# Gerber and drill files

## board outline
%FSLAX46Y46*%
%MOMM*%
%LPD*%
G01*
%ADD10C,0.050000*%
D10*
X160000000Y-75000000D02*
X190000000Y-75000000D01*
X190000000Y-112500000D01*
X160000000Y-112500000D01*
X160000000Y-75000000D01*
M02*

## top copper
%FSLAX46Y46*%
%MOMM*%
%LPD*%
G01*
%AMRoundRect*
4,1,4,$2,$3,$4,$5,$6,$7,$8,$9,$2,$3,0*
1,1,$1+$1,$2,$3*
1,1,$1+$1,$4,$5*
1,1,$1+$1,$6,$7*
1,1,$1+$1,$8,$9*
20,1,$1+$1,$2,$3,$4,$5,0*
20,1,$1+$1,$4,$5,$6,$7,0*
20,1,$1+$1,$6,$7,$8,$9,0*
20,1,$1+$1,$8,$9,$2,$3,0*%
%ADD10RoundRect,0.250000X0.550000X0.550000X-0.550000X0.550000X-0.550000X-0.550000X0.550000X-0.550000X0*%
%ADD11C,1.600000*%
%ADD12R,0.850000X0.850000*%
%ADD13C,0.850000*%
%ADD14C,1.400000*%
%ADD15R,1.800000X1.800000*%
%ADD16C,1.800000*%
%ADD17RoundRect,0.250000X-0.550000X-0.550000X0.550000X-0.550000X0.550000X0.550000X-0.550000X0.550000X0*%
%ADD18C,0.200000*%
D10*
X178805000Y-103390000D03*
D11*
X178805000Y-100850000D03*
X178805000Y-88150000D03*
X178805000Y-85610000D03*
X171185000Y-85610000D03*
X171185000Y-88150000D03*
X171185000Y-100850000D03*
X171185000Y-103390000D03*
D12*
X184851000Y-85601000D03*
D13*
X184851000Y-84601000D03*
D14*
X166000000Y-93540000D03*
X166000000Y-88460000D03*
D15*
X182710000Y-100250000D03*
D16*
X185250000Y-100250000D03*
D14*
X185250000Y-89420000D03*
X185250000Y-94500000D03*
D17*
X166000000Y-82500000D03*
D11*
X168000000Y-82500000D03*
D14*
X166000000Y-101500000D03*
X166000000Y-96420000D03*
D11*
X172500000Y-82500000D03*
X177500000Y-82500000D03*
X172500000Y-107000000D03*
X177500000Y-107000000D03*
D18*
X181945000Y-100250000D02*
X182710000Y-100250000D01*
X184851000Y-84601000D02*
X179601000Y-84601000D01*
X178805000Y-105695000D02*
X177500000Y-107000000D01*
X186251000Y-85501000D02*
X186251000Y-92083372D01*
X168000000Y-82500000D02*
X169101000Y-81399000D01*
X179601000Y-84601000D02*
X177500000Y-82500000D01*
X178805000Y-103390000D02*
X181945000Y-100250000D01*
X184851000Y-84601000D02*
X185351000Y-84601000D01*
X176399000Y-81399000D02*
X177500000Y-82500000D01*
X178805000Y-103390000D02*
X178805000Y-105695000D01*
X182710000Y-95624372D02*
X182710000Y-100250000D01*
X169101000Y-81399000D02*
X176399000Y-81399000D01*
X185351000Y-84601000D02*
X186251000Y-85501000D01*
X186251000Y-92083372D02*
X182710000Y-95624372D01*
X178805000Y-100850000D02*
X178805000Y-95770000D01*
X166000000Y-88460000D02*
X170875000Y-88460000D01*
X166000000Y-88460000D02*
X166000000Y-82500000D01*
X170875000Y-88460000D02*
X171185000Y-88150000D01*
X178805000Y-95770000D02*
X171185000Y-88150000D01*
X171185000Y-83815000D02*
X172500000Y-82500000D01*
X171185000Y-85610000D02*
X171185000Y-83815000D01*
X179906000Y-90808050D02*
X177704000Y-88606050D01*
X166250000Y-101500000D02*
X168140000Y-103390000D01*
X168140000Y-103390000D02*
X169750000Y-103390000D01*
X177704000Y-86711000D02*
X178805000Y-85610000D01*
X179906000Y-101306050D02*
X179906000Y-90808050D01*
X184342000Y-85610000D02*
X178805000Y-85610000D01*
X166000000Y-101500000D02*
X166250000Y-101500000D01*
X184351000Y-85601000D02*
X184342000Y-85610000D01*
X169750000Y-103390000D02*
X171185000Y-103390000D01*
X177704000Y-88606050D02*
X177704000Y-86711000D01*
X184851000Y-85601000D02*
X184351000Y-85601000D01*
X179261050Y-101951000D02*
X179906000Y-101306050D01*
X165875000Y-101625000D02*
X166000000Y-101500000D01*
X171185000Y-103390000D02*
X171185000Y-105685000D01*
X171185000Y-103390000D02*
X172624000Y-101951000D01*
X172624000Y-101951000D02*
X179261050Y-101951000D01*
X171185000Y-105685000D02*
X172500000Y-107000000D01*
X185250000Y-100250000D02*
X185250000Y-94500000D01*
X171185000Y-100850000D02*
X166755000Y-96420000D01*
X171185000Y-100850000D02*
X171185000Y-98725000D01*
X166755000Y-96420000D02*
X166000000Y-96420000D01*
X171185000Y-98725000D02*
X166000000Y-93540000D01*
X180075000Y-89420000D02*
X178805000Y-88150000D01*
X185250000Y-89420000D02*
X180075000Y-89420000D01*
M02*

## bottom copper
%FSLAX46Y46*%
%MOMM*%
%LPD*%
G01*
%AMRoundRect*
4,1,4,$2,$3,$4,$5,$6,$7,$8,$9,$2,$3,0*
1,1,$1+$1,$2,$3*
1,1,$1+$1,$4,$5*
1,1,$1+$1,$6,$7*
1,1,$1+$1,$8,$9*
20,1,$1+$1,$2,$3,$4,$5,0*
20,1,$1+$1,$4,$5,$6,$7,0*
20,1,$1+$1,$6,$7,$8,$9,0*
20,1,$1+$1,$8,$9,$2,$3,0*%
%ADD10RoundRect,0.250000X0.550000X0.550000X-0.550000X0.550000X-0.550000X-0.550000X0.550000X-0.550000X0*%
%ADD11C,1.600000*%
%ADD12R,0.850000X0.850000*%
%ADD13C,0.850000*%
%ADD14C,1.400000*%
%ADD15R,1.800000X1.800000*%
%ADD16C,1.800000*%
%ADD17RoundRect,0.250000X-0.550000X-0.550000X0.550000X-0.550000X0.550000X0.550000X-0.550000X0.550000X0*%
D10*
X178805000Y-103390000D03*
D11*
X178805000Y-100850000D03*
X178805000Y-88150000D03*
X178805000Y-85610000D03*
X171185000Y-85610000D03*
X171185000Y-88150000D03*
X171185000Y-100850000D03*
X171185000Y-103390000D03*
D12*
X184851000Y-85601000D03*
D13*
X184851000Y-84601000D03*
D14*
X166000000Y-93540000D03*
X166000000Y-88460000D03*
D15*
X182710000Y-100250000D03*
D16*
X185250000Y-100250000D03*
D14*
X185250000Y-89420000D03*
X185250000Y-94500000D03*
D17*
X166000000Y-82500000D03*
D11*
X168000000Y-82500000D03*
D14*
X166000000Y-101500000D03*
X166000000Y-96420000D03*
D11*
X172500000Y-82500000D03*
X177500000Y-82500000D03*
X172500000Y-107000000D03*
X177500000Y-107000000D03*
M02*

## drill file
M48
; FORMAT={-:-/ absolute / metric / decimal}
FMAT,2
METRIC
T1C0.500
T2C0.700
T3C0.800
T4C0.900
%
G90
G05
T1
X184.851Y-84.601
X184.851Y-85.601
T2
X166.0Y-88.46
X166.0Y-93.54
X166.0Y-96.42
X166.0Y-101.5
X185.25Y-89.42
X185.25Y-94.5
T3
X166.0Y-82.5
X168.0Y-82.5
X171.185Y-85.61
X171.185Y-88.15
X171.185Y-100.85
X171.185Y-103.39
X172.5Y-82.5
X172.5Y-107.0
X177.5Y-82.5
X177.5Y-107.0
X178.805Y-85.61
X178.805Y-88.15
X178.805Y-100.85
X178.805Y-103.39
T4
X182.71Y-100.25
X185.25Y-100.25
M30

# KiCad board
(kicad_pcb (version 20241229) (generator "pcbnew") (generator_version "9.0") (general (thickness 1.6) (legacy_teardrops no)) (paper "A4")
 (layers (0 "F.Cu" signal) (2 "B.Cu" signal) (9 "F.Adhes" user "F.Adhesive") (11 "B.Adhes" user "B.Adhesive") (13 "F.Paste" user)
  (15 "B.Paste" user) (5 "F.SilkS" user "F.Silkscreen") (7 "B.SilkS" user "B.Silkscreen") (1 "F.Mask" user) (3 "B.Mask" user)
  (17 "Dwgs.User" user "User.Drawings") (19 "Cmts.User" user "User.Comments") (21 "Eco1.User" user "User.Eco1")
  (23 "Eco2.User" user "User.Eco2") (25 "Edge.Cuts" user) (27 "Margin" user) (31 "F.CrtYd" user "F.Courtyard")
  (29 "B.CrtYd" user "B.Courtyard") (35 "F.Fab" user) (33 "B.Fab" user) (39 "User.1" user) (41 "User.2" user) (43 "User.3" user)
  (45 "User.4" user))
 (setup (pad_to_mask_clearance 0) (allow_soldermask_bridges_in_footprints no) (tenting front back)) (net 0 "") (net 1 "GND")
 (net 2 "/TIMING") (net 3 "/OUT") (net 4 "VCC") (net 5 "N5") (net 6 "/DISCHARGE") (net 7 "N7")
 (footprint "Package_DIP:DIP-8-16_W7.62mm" (layer "F.Cu") (at 178.805 103.39 180)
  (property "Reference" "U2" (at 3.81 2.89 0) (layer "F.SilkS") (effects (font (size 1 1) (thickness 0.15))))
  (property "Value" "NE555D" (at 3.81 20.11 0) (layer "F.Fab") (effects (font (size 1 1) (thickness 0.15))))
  (pad "1" thru_hole roundrect (at 0 0 180) (size 1.6 1.6) (drill 0.8) (layers "*.Cu" "*.Mask") (remove_unused_layers no)
   (roundrect_rratio 0.15625) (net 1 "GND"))
  (pad "2" thru_hole circle (at 0 2.54 180) (size 1.6 1.6) (drill 0.8) (layers "*.Cu" "*.Mask") (remove_unused_layers no) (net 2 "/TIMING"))
  (pad "3" thru_hole circle (at 0 15.24 180) (size 1.6 1.6) (drill 0.8) (layers "*.Cu" "*.Mask") (remove_unused_layers no) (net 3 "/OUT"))
  (pad "4" thru_hole circle (at 0 17.78 180) (size 1.6 1.6) (drill 0.8) (layers "*.Cu" "*.Mask") (remove_unused_layers no) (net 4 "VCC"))
  (pad "5" thru_hole circle (at 7.62 17.78 180) (size 1.6 1.6) (drill 0.8) (layers "*.Cu" "*.Mask") (remove_unused_layers no) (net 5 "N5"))
  (pad "6" thru_hole circle (at 7.62 15.24 180) (size 1.6 1.6) (drill 0.8) (layers "*.Cu" "*.Mask") (remove_unused_layers no)
   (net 2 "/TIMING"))
  (pad "7" thru_hole circle (at 7.62 2.54 180) (size 1.6 1.6) (drill 0.8) (layers "*.Cu" "*.Mask") (remove_unused_layers no)
   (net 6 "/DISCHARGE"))
  (pad "8" thru_hole circle (at 7.62 0 180) (size 1.6 1.6) (drill 0.8) (layers "*.Cu" "*.Mask") (remove_unused_layers no) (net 4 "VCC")))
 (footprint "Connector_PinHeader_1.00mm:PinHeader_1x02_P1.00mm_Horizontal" (layer "F.Cu") (at 184.851 85.601 180)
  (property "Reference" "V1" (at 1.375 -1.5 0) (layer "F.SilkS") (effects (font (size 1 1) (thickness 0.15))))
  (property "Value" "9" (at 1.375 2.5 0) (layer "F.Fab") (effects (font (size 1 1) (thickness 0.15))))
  (pad "1" thru_hole rect (at 0 0 180) (size 0.85 0.85) (drill 0.5) (layers "*.Cu" "*.Mask") (remove_unused_layers no) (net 4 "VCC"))
  (pad "2" thru_hole circle (at 0 1 180) (size 0.85 0.85) (drill 0.5) (layers "*.Cu" "*.Mask") (remove_unused_layers no) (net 1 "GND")))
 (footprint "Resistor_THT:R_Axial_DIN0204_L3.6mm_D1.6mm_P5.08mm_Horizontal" (layer "F.Cu") (at 166 93.54 90)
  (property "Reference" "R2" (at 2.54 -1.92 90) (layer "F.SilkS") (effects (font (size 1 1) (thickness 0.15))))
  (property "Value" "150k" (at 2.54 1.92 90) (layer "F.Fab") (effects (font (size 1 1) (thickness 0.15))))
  (pad "1" thru_hole circle (at 0 0 90) (size 1.4 1.4) (drill 0.7) (layers "*.Cu" "*.Mask") (remove_unused_layers no) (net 6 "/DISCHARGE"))
  (pad "2" thru_hole circle (at 5.08 0 90) (size 1.4 1.4) (drill 0.7) (layers "*.Cu" "*.Mask") (remove_unused_layers no) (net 2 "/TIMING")))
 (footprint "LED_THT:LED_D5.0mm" (layer "F.Cu") (at 182.71 100.25)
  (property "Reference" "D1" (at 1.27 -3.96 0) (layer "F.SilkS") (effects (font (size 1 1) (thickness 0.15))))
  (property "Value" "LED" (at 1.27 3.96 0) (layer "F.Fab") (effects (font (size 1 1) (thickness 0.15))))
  (pad "1" thru_hole rect (at 0 0) (size 1.8 1.8) (drill 0.9) (layers "*.Cu" "*.Mask") (remove_unused_layers no) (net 1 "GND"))
  (pad "2" thru_hole circle (at 2.54 0) (size 1.8 1.8) (drill 0.9) (layers "*.Cu" "*.Mask") (remove_unused_layers no) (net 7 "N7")))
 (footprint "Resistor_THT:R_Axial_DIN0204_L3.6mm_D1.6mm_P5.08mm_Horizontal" (layer "F.Cu") (at 185.25 89.42 -90)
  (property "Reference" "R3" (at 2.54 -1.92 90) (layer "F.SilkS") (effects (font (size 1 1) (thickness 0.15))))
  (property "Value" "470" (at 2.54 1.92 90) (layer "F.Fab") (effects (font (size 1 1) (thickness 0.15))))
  (pad "1" thru_hole circle (at 0 0 270) (size 1.4 1.4) (drill 0.7) (layers "*.Cu" "*.Mask") (remove_unused_layers no) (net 3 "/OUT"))
  (pad "2" thru_hole circle (at 5.08 0 270) (size 1.4 1.4) (drill 0.7) (layers "*.Cu" "*.Mask") (remove_unused_layers no) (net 7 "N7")))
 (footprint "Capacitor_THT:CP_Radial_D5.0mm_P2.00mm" (layer "F.Cu") (at 166 82.5)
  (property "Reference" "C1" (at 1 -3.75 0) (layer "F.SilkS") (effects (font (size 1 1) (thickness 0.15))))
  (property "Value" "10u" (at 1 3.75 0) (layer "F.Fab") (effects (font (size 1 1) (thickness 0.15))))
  (pad "1" thru_hole roundrect (at 0 0) (size 1.6 1.6) (drill 0.8) (layers "*.Cu" "*.Mask") (remove_unused_layers no)
   (roundrect_rratio 0.15625) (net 2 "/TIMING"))
  (pad "2" thru_hole circle (at 2 0) (size 1.6 1.6) (drill 0.8) (layers "*.Cu" "*.Mask") (remove_unused_layers no) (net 1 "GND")))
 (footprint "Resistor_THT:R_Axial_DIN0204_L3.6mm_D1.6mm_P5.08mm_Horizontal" (layer "F.Cu") (at 166 101.5 90)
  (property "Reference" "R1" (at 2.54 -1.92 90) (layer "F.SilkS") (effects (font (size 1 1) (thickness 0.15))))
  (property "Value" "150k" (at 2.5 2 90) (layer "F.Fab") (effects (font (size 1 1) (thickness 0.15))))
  (pad "1" thru_hole circle (at 0 0 90) (size 1.4 1.4) (drill 0.7) (layers "*.Cu" "*.Mask") (remove_unused_layers no) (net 4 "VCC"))
  (pad "2" thru_hole circle (at 5.08 0 90) (size 1.4 1.4) (drill 0.7) (layers "*.Cu" "*.Mask") (remove_unused_layers no)
   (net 6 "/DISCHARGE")))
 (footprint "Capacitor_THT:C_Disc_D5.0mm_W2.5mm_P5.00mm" (layer "F.Cu") (at 172.5 82.5)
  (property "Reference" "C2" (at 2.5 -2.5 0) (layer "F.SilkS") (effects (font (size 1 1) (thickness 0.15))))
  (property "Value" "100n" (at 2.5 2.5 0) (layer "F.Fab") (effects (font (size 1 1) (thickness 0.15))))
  (pad "1" thru_hole circle (at 0 0) (size 1.6 1.6) (drill 0.8) (layers "*.Cu" "*.Mask") (remove_unused_layers no) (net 5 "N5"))
  (pad "2" thru_hole circle (at 5 0) (size 1.6 1.6) (drill 0.8) (layers "*.Cu" "*.Mask") (remove_unused_layers no) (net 1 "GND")))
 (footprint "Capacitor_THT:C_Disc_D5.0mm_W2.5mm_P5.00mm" (layer "F.Cu") (at 172.5 107)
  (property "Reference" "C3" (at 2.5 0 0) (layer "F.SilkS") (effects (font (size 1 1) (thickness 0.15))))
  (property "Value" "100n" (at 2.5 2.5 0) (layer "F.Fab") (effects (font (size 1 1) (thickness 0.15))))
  (pad "1" thru_hole circle (at 0 0) (size 1.6 1.6) (drill 0.8) (layers "*.Cu" "*.Mask") (remove_unused_layers no) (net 4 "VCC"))
  (pad "2" thru_hole circle (at 5 0) (size 1.6 1.6) (drill 0.8) (layers "*.Cu" "*.Mask") (remove_unused_layers no) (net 1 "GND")))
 (gr_rect (start 160 75) (end 190 112.5) (stroke (width 0.05) (type default)) (fill no) (layer "Edge.Cuts"))
 (segment (start 181.945 100.25) (end 182.71 100.25) (width 0.2) (layer "F.Cu") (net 1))
 (segment (start 184.851 84.601) (end 179.601 84.601) (width 0.2) (layer "F.Cu") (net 1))
 (segment (start 178.805 105.695) (end 177.5 107) (width 0.2) (layer "F.Cu") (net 1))
 (segment (start 186.251 85.501) (end 186.251 92.083372) (width 0.2) (layer "F.Cu") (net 1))
 (segment (start 168 82.5) (end 169.101 81.399) (width 0.2) (layer "F.Cu") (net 1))
 (segment (start 179.601 84.601) (end 177.5 82.5) (width 0.2) (layer "F.Cu") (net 1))
 (segment (start 178.805 103.39) (end 181.945 100.25) (width 0.2) (layer "F.Cu") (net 1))
 (segment (start 184.851 84.601) (end 185.351 84.601) (width 0.2) (layer "F.Cu") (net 1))
 (segment (start 176.399 81.399) (end 177.5 82.5) (width 0.2) (layer "F.Cu") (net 1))
 (segment (start 178.805 103.39) (end 178.805 105.695) (width 0.2) (layer "F.Cu") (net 1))
 (segment (start 182.71 95.624372) (end 182.71 100.25) (width 0.2) (layer "F.Cu") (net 1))
 (segment (start 169.101 81.399) (end 176.399 81.399) (width 0.2) (layer "F.Cu") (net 1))
 (segment (start 185.351 84.601) (end 186.251 85.501) (width 0.2) (layer "F.Cu") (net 1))
 (segment (start 186.251 92.083372) (end 182.71 95.624372) (width 0.2) (layer "F.Cu") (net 1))
 (segment (start 178.805 100.85) (end 178.805 95.77) (width 0.2) (layer "F.Cu") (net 2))
 (segment (start 166 88.46) (end 170.875 88.46) (width 0.2) (layer "F.Cu") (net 2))
 (segment (start 166 88.46) (end 166 82.5) (width 0.2) (layer "F.Cu") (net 2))
 (segment (start 170.875 88.46) (end 171.185 88.15) (width 0.2) (layer "F.Cu") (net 2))
 (segment (start 178.805 95.77) (end 171.185 88.15) (width 0.2) (layer "F.Cu") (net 2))
 (segment (start 171.185 83.815) (end 172.5 82.5) (width 0.2) (layer "F.Cu") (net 5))
 (segment (start 171.185 85.61) (end 171.185 83.815) (width 0.2) (layer "F.Cu") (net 5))
 (segment (start 179.906 90.80805) (end 177.704 88.60605) (width 0.2) (layer "F.Cu") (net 4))
 (segment (start 166.25 101.5) (end 168.14 103.39) (width 0.2) (layer "F.Cu") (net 4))
 (segment (start 168.14 103.39) (end 169.75 103.39) (width 0.2) (layer "F.Cu") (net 4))
 (segment (start 177.704 86.711) (end 178.805 85.61) (width 0.2) (layer "F.Cu") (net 4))
 (segment (start 179.906 101.30605) (end 179.906 90.80805) (width 0.2) (layer "F.Cu") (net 4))
 (segment (start 184.342 85.61) (end 178.805 85.61) (width 0.2) (layer "F.Cu") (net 4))
 (segment (start 166 101.5) (end 166.25 101.5) (width 0.2) (layer "F.Cu") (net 4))
 (segment (start 184.351 85.601) (end 184.342 85.61) (width 0.2) (layer "F.Cu") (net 4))
 (segment (start 169.75 103.39) (end 171.185 103.39) (width 0.2) (layer "F.Cu") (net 4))
 (segment (start 177.704 88.60605) (end 177.704 86.711) (width 0.2) (layer "F.Cu") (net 4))
 (segment (start 184.851 85.601) (end 184.351 85.601) (width 0.2) (layer "F.Cu") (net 4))
 (segment (start 179.26105 101.951) (end 179.906 101.30605) (width 0.2) (layer "F.Cu") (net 4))
 (segment (start 165.875 101.625) (end 166 101.5) (width 0.2) (layer "F.Cu") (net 4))
 (segment (start 171.185 103.39) (end 171.185 105.685) (width 0.2) (layer "F.Cu") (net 4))
 (segment (start 171.185 103.39) (end 172.624 101.951) (width 0.2) (layer "F.Cu") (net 4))
 (segment (start 172.624 101.951) (end 179.26105 101.951) (width 0.2) (layer "F.Cu") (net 4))
 (segment (start 171.185 105.685) (end 172.5 107) (width 0.2) (layer "F.Cu") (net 4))
 (segment (start 185.25 100.25) (end 185.25 94.5) (width 0.2) (layer "F.Cu") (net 7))
 (segment (start 171.185 100.85) (end 166.755 96.42) (width 0.2) (layer "F.Cu") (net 6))
 (segment (start 171.185 100.85) (end 171.185 98.725) (width 0.2) (layer "F.Cu") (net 6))
 (segment (start 166.755 96.42) (end 166 96.42) (width 0.2) (layer "F.Cu") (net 6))
 (segment (start 171.185 98.725) (end 166 93.54) (width 0.2) (layer "F.Cu") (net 6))
 (segment (start 180.075 89.42) (end 178.805 88.15) (width 0.2) (layer "F.Cu") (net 3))
 (segment (start 185.25 89.42) (end 180.075 89.42) (width 0.2) (layer "F.Cu") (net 3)))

